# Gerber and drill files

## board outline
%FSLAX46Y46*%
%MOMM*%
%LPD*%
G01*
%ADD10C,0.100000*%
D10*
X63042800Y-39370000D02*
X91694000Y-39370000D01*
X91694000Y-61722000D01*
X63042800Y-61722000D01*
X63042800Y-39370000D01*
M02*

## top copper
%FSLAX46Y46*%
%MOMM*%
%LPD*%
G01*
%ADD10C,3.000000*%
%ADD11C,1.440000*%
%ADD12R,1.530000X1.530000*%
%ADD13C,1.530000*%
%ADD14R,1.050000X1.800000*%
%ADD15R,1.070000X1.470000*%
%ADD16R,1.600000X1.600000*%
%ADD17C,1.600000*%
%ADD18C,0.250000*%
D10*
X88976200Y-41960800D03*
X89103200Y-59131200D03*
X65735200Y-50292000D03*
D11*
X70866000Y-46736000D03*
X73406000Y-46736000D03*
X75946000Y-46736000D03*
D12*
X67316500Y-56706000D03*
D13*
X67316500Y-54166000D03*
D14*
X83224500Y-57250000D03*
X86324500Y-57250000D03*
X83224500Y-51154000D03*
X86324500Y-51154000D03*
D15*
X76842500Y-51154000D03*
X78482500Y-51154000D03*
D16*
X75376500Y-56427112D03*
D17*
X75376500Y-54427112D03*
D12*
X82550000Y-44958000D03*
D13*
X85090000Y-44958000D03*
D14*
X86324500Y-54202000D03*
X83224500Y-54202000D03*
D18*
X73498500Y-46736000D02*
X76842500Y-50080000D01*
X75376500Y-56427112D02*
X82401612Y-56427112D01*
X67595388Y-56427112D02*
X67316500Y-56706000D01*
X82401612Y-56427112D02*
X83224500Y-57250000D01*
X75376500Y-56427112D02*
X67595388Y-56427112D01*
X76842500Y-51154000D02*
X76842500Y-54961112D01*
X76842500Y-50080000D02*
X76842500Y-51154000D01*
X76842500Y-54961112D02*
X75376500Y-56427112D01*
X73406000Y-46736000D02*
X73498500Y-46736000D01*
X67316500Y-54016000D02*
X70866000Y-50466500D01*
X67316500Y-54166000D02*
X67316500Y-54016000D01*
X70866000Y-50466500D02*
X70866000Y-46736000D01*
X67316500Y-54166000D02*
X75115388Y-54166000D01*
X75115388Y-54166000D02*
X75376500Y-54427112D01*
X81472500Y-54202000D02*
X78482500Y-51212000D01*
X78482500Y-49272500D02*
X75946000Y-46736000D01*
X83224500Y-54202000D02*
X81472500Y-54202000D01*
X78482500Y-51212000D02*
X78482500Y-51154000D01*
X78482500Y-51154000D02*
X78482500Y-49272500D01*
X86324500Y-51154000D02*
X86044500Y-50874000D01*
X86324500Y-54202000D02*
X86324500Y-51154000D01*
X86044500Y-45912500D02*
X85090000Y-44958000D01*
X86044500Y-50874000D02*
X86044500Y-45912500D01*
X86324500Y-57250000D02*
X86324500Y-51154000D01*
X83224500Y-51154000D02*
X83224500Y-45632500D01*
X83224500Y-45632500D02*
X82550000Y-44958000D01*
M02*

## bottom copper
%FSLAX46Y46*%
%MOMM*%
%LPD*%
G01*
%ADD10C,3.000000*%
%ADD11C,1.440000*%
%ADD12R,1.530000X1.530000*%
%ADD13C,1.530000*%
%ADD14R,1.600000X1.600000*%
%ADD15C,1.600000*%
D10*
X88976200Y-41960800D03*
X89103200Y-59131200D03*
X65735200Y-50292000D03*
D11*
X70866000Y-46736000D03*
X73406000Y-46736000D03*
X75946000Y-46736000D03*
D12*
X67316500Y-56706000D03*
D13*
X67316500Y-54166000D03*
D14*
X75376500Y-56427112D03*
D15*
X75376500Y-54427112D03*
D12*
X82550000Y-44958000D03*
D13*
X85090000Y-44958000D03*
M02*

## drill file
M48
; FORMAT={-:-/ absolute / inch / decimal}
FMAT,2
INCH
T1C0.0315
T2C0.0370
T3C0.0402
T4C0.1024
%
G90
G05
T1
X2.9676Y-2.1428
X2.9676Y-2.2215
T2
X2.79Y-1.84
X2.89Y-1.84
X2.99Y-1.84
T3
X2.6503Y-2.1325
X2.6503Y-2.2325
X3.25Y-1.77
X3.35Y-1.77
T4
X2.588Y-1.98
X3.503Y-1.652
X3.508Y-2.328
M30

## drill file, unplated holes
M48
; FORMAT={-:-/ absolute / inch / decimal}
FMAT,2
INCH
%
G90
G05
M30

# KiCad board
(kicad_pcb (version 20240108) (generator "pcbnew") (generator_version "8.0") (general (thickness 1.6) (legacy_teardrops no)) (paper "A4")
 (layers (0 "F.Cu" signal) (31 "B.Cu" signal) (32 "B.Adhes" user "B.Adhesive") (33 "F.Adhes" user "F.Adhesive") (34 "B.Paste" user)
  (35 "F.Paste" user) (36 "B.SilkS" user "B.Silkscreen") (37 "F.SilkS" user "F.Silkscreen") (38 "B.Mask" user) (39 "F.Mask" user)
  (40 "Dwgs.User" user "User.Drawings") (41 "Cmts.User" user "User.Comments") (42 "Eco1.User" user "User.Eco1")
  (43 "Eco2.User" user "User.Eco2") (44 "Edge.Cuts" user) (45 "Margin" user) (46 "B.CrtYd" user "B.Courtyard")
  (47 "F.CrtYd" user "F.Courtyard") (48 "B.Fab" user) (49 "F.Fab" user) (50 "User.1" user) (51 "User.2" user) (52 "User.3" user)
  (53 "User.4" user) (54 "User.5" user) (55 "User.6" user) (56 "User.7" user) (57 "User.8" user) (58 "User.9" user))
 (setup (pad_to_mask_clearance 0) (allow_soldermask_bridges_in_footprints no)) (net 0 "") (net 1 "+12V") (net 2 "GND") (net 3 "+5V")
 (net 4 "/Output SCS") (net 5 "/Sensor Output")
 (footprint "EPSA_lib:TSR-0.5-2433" (layer "F.Cu") (at 67.656 48.736)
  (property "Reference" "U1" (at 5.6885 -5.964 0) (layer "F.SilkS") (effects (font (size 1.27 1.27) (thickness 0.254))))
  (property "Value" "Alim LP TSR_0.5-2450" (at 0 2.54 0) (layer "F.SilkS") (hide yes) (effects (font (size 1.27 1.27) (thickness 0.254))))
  (pad "1" thru_hole circle (at 3.21 -2) (size 1.44 1.44) (drill 0.94) (layers "*.Cu" "*.Mask") (remove_unused_layers no) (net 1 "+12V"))
  (pad "2" thru_hole circle (at 5.75 -2) (size 1.44 1.44) (drill 0.94) (layers "*.Cu" "*.Mask") (remove_unused_layers no) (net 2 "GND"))
  (pad "3" thru_hole circle (at 8.29 -2) (size 1.44 1.44) (drill 0.94) (layers "*.Cu" "*.Mask") (remove_unused_layers no) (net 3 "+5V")))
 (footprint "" (layer "F.Cu") (at 88.9762 41.9608)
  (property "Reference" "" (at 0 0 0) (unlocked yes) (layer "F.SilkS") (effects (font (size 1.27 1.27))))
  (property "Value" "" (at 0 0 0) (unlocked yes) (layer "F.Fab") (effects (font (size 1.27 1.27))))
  (pad "1" thru_hole circle (at 0 0) (size 3 3) (drill 2.6) (layers "*.Cu" "*.Mask") (remove_unused_layers no)))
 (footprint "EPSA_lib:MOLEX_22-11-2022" (layer "F.Cu") (at 67.3165 56.706 90)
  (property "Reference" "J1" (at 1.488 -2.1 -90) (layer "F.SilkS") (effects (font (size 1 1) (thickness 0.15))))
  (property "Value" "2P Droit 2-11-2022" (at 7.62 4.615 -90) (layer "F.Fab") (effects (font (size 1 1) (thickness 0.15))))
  (pad "1" thru_hole rect (at 0 0 90) (size 1.53 1.53) (drill 1.02) (layers "*.Cu" "*.Mask") (remove_unused_layers no) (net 2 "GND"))
  (pad "2" thru_hole circle (at 2.54 0 90) (size 1.53 1.53) (drill 1.02) (layers "*.Cu" "*.Mask") (remove_unused_layers no) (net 1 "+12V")))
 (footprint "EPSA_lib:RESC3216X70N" (layer "F.Cu") (at 84.7745 57.25)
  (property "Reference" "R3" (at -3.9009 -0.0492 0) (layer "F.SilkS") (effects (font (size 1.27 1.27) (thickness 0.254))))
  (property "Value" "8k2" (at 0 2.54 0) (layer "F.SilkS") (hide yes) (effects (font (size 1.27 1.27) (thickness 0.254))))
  (pad "1" smd rect (at -1.55 0) (size 1.05 1.8) (layers "F.Cu" "F.Paste" "F.Mask") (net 2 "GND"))
  (pad "2" smd rect (at 1.55 0) (size 1.05 1.8) (layers "F.Cu" "F.Paste" "F.Mask") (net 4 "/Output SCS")))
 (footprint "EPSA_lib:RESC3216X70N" (layer "F.Cu") (at 84.7745 51.154)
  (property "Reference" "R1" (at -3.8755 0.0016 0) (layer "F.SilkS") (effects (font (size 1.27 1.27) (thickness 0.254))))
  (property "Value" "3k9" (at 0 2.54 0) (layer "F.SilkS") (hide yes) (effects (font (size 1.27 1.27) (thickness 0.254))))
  (pad "1" smd rect (at -1.55 0) (size 1.05 1.8) (layers "F.Cu" "F.Paste" "F.Mask") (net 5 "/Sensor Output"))
  (pad "2" smd rect (at 1.55 0) (size 1.05 1.8) (layers "F.Cu" "F.Paste" "F.Mask") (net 4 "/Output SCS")))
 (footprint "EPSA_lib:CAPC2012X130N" (layer "F.Cu") (at 77.6625 51.154)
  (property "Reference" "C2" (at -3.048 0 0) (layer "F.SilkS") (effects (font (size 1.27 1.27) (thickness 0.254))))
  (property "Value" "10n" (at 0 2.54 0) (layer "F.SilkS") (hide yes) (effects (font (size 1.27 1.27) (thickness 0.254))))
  (pad "1" smd rect (at -0.82 0) (size 1.07 1.47) (layers "F.Cu" "F.Paste" "F.Mask") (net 2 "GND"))
  (pad "2" smd rect (at 0.82 0) (size 1.07 1.47) (layers "F.Cu" "F.Paste" "F.Mask") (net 3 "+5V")))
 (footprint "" (layer "F.Cu") (at 89.1032 59.1312)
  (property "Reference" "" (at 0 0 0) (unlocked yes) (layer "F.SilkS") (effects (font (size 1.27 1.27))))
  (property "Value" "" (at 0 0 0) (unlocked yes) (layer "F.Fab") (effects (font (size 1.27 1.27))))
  (pad "1" thru_hole circle (at 0 0) (size 3 3) (drill 2.6) (layers "*.Cu" "*.Mask") (remove_unused_layers no)))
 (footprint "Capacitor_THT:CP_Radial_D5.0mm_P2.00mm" (layer "F.Cu") (at 75.3765 56.427112 90)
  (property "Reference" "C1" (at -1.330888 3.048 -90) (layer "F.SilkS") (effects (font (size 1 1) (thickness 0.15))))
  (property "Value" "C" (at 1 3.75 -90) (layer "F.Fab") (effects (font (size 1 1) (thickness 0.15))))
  (pad "1" thru_hole rect (at 0 0 90) (size 1.6 1.6) (drill 0.8) (layers "*.Cu" "*.Mask") (remove_unused_layers no) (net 2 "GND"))
  (pad "2" thru_hole circle (at 2 0 90) (size 1.6 1.6) (drill 0.8) (layers "*.Cu" "*.Mask") (remove_unused_layers no) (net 1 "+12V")))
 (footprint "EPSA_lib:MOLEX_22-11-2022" (layer "F.Cu") (at 82.55 44.958)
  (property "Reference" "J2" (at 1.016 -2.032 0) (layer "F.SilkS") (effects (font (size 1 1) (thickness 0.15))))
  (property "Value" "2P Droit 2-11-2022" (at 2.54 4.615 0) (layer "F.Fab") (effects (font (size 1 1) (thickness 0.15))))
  (pad "1" thru_hole rect (at 0 0) (size 1.53 1.53) (drill 1.02) (layers "*.Cu" "*.Mask") (remove_unused_layers no) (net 5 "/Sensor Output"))
  (pad "2" thru_hole circle (at 2.54 0) (size 1.53 1.53) (drill 1.02) (layers "*.Cu" "*.Mask") (remove_unused_layers no)
   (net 4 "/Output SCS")))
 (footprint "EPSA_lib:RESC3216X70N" (layer "F.Cu") (at 84.7745 54.202 180)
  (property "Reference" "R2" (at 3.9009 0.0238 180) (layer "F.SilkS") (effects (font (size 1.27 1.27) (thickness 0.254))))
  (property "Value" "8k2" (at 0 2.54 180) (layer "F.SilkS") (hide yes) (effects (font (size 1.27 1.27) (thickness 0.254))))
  (pad "1" smd rect (at -1.55 0 180) (size 1.05 1.8) (layers "F.Cu" "F.Paste" "F.Mask") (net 4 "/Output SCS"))
  (pad "2" smd rect (at 1.55 0 180) (size 1.05 1.8) (layers "F.Cu" "F.Paste" "F.Mask") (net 3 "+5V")))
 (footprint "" (layer "F.Cu") (at 65.7352 50.292)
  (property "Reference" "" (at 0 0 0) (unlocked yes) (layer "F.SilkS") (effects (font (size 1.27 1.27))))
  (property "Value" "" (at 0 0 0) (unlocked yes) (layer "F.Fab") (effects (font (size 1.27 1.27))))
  (pad "1" thru_hole circle (at 0 0) (size 3 3) (drill 2.6) (layers "*.Cu" "*.Mask") (remove_unused_layers no)))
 (gr_rect (start 63.0428 39.37) (end 91.694 61.722) (stroke (width 0.1) (type default)) (fill none) (layer "Edge.Cuts"))
 (segment (start 73.4985 46.736) (end 76.8425 50.08) (width 0.25) (layer "F.Cu") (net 2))
 (segment (start 75.3765 56.427112) (end 82.401612 56.427112) (width 0.25) (layer "F.Cu") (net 2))
 (segment (start 67.595388 56.427112) (end 67.3165 56.706) (width 0.25) (layer "F.Cu") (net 2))
 (segment (start 82.401612 56.427112) (end 83.2245 57.25) (width 0.25) (layer "F.Cu") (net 2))
 (segment (start 75.3765 56.427112) (end 67.595388 56.427112) (width 0.25) (layer "F.Cu") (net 2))
 (segment (start 76.8425 51.154) (end 76.8425 54.961112) (width 0.25) (layer "F.Cu") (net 2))
 (segment (start 76.8425 50.08) (end 76.8425 51.154) (width 0.25) (layer "F.Cu") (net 2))
 (segment (start 76.8425 54.961112) (end 75.3765 56.427112) (width 0.25) (layer "F.Cu") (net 2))
 (segment (start 73.406 46.736) (end 73.4985 46.736) (width 0.25) (layer "F.Cu") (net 2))
 (segment (start 67.3165 54.016) (end 70.866 50.4665) (width 0.25) (layer "F.Cu") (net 1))
 (segment (start 67.3165 54.166) (end 67.3165 54.016) (width 0.25) (layer "F.Cu") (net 1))
 (segment (start 70.866 50.4665) (end 70.866 46.736) (width 0.25) (layer "F.Cu") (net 1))
 (segment (start 67.3165 54.166) (end 75.115388 54.166) (width 0.25) (layer "F.Cu") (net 1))
 (segment (start 75.115388 54.166) (end 75.3765 54.427112) (width 0.25) (layer "F.Cu") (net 1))
 (segment (start 81.4725 54.202) (end 78.4825 51.212) (width 0.25) (layer "F.Cu") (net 3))
 (segment (start 78.4825 49.2725) (end 75.946 46.736) (width 0.25) (layer "F.Cu") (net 3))
 (segment (start 83.2245 54.202) (end 81.4725 54.202) (width 0.25) (layer "F.Cu") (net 3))
 (segment (start 78.4825 51.212) (end 78.4825 51.154) (width 0.25) (layer "F.Cu") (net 3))
 (segment (start 78.4825 51.154) (end 78.4825 49.2725) (width 0.25) (layer "F.Cu") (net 3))
 (segment (start 86.3245 51.154) (end 86.0445 50.874) (width 0.25) (layer "F.Cu") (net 4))
 (segment (start 86.3245 54.202) (end 86.3245 51.154) (width 0.25) (layer "F.Cu") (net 4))
 (segment (start 86.0445 45.9125) (end 85.09 44.958) (width 0.25) (layer "F.Cu") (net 4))
 (segment (start 86.0445 50.874) (end 86.0445 45.9125) (width 0.25) (layer "F.Cu") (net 4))
 (segment (start 86.3245 57.25) (end 86.3245 51.154) (width 0.25) (layer "F.Cu") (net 4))
 (segment (start 83.2245 51.154) (end 83.2245 45.6325) (width 0.25) (layer "F.Cu") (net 5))
 (segment (start 83.2245 45.6325) (end 82.55 44.958) (width 0.25) (layer "F.Cu") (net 5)))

